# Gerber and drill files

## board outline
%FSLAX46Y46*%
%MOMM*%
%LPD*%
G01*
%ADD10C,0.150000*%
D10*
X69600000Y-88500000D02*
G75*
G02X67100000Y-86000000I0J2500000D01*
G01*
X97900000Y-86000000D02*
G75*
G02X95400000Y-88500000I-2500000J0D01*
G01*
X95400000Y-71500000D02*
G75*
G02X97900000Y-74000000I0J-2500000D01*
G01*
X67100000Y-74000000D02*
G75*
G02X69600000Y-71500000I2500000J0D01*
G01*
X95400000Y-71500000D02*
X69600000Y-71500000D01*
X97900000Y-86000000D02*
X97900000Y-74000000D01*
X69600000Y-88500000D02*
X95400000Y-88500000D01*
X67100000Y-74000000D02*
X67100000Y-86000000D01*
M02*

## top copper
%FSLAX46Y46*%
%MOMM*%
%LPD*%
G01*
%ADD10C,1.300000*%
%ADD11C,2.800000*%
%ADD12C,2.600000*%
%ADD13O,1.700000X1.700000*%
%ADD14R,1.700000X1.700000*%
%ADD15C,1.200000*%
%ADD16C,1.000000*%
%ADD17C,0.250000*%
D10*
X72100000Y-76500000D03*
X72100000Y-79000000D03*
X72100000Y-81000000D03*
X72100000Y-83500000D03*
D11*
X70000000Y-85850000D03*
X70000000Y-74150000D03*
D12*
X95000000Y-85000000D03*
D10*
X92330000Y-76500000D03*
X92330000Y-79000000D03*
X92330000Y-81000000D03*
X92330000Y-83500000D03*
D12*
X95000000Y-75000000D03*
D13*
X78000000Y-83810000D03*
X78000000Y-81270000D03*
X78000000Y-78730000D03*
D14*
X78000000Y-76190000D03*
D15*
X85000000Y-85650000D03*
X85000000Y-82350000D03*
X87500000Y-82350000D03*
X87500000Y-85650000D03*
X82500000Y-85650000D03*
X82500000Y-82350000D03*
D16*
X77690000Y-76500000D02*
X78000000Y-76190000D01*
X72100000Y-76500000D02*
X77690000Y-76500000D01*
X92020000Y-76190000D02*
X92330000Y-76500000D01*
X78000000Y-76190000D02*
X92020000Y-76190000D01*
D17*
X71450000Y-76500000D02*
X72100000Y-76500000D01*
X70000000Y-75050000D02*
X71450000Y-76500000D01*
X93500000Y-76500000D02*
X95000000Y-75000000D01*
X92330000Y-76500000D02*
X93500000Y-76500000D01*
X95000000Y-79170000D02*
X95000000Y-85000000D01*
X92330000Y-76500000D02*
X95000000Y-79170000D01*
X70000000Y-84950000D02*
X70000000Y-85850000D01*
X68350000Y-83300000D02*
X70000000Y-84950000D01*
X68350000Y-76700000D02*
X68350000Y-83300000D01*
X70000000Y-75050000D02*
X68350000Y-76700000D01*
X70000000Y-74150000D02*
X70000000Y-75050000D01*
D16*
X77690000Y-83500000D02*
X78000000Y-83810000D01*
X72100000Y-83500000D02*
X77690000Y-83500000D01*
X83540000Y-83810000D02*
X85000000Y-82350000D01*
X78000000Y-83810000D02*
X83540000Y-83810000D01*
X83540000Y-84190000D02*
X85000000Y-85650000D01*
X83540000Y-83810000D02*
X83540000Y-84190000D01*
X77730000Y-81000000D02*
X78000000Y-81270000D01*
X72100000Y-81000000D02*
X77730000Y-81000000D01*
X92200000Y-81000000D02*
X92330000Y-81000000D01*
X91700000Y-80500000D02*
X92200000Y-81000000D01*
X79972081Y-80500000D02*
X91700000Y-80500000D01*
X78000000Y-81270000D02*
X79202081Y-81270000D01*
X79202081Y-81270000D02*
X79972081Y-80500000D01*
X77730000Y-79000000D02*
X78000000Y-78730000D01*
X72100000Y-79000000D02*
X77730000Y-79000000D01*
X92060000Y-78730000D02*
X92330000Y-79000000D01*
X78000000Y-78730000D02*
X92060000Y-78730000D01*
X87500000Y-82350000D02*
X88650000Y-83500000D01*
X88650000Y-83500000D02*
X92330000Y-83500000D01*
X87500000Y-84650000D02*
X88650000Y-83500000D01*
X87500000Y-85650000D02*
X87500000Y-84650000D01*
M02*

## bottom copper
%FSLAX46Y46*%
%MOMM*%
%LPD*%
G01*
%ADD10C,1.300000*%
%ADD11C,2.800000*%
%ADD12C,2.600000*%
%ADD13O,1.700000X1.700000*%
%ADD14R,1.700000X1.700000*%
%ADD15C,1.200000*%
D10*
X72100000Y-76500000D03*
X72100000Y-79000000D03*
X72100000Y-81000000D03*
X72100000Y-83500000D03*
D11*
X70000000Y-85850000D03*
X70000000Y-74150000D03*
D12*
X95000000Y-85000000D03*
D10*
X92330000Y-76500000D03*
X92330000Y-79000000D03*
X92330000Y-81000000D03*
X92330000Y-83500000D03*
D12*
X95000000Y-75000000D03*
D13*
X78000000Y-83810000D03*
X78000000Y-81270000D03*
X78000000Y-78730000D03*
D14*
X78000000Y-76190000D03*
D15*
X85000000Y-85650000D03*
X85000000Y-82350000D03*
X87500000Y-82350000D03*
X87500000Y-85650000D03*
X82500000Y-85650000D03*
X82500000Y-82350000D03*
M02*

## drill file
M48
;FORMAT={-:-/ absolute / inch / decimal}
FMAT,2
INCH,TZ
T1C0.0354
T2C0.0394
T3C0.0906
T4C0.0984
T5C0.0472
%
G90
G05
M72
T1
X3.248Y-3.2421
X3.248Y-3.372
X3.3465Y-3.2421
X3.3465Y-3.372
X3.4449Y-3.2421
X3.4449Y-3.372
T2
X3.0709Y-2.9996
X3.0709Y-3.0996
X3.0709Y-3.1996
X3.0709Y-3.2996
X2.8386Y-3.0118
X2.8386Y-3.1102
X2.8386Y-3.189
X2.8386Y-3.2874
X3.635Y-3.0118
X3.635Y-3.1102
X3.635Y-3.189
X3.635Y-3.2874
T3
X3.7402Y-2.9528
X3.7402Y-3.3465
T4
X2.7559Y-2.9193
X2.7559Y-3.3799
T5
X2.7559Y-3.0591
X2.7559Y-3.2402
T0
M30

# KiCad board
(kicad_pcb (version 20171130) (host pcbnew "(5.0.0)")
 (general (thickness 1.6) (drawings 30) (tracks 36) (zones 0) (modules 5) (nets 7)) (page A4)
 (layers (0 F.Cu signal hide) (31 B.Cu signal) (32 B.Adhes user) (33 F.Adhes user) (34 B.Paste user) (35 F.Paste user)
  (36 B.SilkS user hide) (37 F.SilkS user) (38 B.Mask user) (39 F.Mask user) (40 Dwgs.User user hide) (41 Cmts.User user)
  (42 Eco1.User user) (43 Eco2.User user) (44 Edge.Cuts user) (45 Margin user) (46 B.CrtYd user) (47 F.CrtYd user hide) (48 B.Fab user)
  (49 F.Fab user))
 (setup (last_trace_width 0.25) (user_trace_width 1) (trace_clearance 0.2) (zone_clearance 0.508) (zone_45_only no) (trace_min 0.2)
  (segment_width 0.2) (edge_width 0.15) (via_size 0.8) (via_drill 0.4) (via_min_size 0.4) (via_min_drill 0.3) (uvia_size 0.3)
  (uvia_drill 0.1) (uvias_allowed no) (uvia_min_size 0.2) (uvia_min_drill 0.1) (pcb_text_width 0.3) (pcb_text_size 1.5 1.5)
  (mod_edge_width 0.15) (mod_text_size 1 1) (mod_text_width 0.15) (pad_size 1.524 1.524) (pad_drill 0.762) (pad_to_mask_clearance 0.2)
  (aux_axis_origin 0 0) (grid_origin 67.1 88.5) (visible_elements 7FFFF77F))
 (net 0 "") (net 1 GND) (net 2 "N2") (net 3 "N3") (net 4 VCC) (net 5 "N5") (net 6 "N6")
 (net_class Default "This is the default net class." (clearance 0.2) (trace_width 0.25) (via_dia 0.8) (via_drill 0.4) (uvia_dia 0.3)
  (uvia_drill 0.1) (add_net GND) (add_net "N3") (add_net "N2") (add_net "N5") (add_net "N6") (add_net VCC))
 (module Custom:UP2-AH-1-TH (layer F.Cu) (at 70 80 270)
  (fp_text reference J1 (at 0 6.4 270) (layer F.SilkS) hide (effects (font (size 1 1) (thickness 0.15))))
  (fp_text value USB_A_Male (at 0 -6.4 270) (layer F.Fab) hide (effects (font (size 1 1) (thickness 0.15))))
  (pad 4 thru_hole circle (at -3.5 -2.1 270) (size 1.3 1.3) (drill 1) (layers *.Cu *.Mask) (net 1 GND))
  (pad 3 thru_hole circle (at -1 -2.1 270) (size 1.3 1.3) (drill 1) (layers *.Cu *.Mask) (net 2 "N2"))
  (pad 2 thru_hole circle (at 1 -2.1 270) (size 1.3 1.3) (drill 1) (layers *.Cu *.Mask) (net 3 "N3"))
  (pad 1 thru_hole circle (at 3.5 -2.1 270) (size 1.3 1.3) (drill 1) (layers *.Cu *.Mask) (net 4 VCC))
  (pad 5 thru_hole circle (at 5.85 0 270) (size 2.8 2.8) (drill 2.5) (layers *.Cu *.Mask) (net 1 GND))
  (pad 5 thru_hole circle (at -5.85 0 270) (size 2.8 2.8) (drill 2.5) (layers *.Cu *.Mask) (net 1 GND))
  (pad "" np_thru_hole circle (at 2.3 0 270) (size 1.2 1.2) (drill 1.2) (layers *.Cu *.Mask))
  (pad "" np_thru_hole circle (at -2.3 0 270) (size 1.2 1.2) (drill 1.2) (layers *.Cu *.Mask)))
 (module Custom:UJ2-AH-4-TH (layer F.Cu) (at 95 80 90)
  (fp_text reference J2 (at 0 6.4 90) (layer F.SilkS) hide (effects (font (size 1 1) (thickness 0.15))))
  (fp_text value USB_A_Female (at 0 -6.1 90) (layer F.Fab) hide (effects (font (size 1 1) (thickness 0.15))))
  (pad 5 thru_hole circle (at -5 0 90) (size 2.6 2.6) (drill 2.3) (layers *.Cu *.Mask) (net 1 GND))
  (pad 4 thru_hole circle (at 3.5 -2.67 90) (size 1.3 1.3) (drill 1) (layers *.Cu *.Mask) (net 1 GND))
  (pad 3 thru_hole circle (at 1 -2.67 90) (size 1.3 1.3) (drill 1) (layers *.Cu *.Mask) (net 2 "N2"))
  (pad 2 thru_hole circle (at -1 -2.67 90) (size 1.3 1.3) (drill 1) (layers *.Cu *.Mask) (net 3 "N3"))
  (pad 1 thru_hole circle (at -3.5 -2.67 90) (size 1.3 1.3) (drill 1) (layers *.Cu *.Mask) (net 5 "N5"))
  (pad 5 thru_hole circle (at 5 0 90) (size 2.6 2.6) (drill 2.3) (layers *.Cu *.Mask) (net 1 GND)))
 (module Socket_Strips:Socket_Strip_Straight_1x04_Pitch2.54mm (layer F.Cu) (at 78 76.19)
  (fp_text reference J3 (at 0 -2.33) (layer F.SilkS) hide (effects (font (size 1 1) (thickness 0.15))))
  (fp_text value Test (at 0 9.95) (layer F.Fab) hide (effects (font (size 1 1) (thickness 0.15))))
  (pad 4 thru_hole oval (at 0 7.62) (size 1.7 1.7) (drill 1) (layers *.Cu *.Mask) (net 4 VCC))
  (pad 3 thru_hole oval (at 0 5.08) (size 1.7 1.7) (drill 1) (layers *.Cu *.Mask) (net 3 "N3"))
  (pad 2 thru_hole oval (at 0 2.54) (size 1.7 1.7) (drill 1) (layers *.Cu *.Mask) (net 2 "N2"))
  (pad 1 thru_hole rect (at 0 0) (size 1.7 1.7) (drill 1) (layers *.Cu *.Mask) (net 1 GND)))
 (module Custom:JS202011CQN (layer F.Cu) (at 85 84)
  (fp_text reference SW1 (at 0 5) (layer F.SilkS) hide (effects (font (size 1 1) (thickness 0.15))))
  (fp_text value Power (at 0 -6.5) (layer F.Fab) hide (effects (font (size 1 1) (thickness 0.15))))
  (pad 2 thru_hole circle (at 0 1.65) (size 1.2 1.2) (drill 0.9) (layers *.Cu *.Mask) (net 4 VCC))
  (pad 2 thru_hole circle (at 0 -1.65) (size 1.2 1.2) (drill 0.9) (layers *.Cu *.Mask) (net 4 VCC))
  (pad 3 thru_hole circle (at 2.5 -1.65) (size 1.2 1.2) (drill 0.9) (layers *.Cu *.Mask) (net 5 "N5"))
  (pad 3 thru_hole circle (at 2.5 1.65) (size 1.2 1.2) (drill 0.9) (layers *.Cu *.Mask) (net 5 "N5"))
  (pad 1 thru_hole circle (at -2.5 1.65) (size 1.2 1.2) (drill 0.9) (layers *.Cu *.Mask) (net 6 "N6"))
  (pad 1 thru_hole circle (at -2.5 -1.65) (size 1.2 1.2) (drill 0.9) (layers *.Cu *.Mask) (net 6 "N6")))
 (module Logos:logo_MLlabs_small (layer F.Cu) (at 86.9 76.5)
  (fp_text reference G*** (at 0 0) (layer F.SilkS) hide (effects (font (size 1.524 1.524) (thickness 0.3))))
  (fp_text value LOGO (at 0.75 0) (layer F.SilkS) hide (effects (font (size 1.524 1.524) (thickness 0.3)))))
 (gr_arc (start 69.6 86) (end 67.1 86) (angle -90) (layer Edge.Cuts) (width 0.15))
 (gr_arc (start 95.4 86) (end 95.4 88.5) (angle -90) (layer Edge.Cuts) (width 0.15))
 (gr_arc (start 95.4 74) (end 97.9 74) (angle -90) (layer Edge.Cuts) (width 0.15))
 (gr_arc (start 69.6 74) (end 69.6 71.5) (angle -90) (layer Edge.Cuts) (width 0.15))
 (gr_line (start 95.4 71.5) (end 69.6 71.5) (layer Edge.Cuts) (width 0.15))
 (gr_line (start 97.9 86) (end 97.9 74) (layer Edge.Cuts) (width 0.15))
 (gr_line (start 69.6 88.5) (end 95.4 88.5) (layer Edge.Cuts) (width 0.15))
 (gr_line (start 67.1 74) (end 67.1 86) (layer Edge.Cuts) (width 0.15))
 (segment (start 77.69 76.5) (end 78 76.19) (width 1) (layer F.Cu) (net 1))
 (segment (start 72.1 76.5) (end 77.69 76.5) (width 1) (layer F.Cu) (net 1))
 (segment (start 92.02 76.19) (end 92.33 76.5) (width 1) (layer F.Cu) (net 1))
 (segment (start 78 76.19) (end 92.02 76.19) (width 1) (layer F.Cu) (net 1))
 (segment (start 71.45 76.5) (end 72.1 76.5) (width 0.25) (layer F.Cu) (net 1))
 (segment (start 70 75.05) (end 71.45 76.5) (width 0.25) (layer F.Cu) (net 1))
 (segment (start 93.5 76.5) (end 95 75) (width 0.25) (layer F.Cu) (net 1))
 (segment (start 92.33 76.5) (end 93.5 76.5) (width 0.25) (layer F.Cu) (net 1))
 (segment (start 95 79.17) (end 95 85) (width 0.25) (layer F.Cu) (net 1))
 (segment (start 92.33 76.5) (end 95 79.17) (width 0.25) (layer F.Cu) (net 1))
 (segment (start 70 84.95) (end 70 85.85) (width 0.25) (layer F.Cu) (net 1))
 (segment (start 68.35 83.3) (end 70 84.95) (width 0.25) (layer F.Cu) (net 1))
 (segment (start 68.35 76.7) (end 68.35 83.3) (width 0.25) (layer F.Cu) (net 1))
 (segment (start 70 75.05) (end 68.35 76.7) (width 0.25) (layer F.Cu) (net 1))
 (segment (start 70 74.15) (end 70 75.05) (width 0.25) (layer F.Cu) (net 1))
 (segment (start 77.69 83.5) (end 78 83.81) (width 1) (layer F.Cu) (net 4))
 (segment (start 72.1 83.5) (end 77.69 83.5) (width 1) (layer F.Cu) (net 4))
 (segment (start 83.54 83.81) (end 85 82.35) (width 1) (layer F.Cu) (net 4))
 (segment (start 78 83.81) (end 83.54 83.81) (width 1) (layer F.Cu) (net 4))
 (segment (start 83.54 84.19) (end 85 85.65) (width 1) (layer F.Cu) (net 4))
 (segment (start 83.54 83.81) (end 83.54 84.19) (width 1) (layer F.Cu) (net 4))
 (segment (start 77.73 81) (end 78 81.27) (width 1) (layer F.Cu) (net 3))
 (segment (start 72.1 81) (end 77.73 81) (width 1) (layer F.Cu) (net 3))
 (segment (start 92.2 81) (end 92.33 81) (width 1) (layer F.Cu) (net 3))
 (segment (start 91.7 80.5) (end 92.2 81) (width 1) (layer F.Cu) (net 3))
 (segment (start 79.972081 80.5) (end 91.7 80.5) (width 1) (layer F.Cu) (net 3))
 (segment (start 78 81.27) (end 79.202081 81.27) (width 1) (layer F.Cu) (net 3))
 (segment (start 79.202081 81.27) (end 79.972081 80.5) (width 1) (layer F.Cu) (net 3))
 (segment (start 77.73 79) (end 78 78.73) (width 1) (layer F.Cu) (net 2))
 (segment (start 72.1 79) (end 77.73 79) (width 1) (layer F.Cu) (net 2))
 (segment (start 92.06 78.73) (end 92.33 79) (width 1) (layer F.Cu) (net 2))
 (segment (start 78 78.73) (end 92.06 78.73) (width 1) (layer F.Cu) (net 2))
 (segment (start 87.5 82.35) (end 88.65 83.5) (width 1) (layer F.Cu) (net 5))
 (segment (start 88.65 83.5) (end 92.33 83.5) (width 1) (layer F.Cu) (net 5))
 (segment (start 87.5 84.65) (end 88.65 83.5) (width 1) (layer F.Cu) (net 5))
 (segment (start 87.5 85.65) (end 87.5 84.65) (width 1) (layer F.Cu) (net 5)))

